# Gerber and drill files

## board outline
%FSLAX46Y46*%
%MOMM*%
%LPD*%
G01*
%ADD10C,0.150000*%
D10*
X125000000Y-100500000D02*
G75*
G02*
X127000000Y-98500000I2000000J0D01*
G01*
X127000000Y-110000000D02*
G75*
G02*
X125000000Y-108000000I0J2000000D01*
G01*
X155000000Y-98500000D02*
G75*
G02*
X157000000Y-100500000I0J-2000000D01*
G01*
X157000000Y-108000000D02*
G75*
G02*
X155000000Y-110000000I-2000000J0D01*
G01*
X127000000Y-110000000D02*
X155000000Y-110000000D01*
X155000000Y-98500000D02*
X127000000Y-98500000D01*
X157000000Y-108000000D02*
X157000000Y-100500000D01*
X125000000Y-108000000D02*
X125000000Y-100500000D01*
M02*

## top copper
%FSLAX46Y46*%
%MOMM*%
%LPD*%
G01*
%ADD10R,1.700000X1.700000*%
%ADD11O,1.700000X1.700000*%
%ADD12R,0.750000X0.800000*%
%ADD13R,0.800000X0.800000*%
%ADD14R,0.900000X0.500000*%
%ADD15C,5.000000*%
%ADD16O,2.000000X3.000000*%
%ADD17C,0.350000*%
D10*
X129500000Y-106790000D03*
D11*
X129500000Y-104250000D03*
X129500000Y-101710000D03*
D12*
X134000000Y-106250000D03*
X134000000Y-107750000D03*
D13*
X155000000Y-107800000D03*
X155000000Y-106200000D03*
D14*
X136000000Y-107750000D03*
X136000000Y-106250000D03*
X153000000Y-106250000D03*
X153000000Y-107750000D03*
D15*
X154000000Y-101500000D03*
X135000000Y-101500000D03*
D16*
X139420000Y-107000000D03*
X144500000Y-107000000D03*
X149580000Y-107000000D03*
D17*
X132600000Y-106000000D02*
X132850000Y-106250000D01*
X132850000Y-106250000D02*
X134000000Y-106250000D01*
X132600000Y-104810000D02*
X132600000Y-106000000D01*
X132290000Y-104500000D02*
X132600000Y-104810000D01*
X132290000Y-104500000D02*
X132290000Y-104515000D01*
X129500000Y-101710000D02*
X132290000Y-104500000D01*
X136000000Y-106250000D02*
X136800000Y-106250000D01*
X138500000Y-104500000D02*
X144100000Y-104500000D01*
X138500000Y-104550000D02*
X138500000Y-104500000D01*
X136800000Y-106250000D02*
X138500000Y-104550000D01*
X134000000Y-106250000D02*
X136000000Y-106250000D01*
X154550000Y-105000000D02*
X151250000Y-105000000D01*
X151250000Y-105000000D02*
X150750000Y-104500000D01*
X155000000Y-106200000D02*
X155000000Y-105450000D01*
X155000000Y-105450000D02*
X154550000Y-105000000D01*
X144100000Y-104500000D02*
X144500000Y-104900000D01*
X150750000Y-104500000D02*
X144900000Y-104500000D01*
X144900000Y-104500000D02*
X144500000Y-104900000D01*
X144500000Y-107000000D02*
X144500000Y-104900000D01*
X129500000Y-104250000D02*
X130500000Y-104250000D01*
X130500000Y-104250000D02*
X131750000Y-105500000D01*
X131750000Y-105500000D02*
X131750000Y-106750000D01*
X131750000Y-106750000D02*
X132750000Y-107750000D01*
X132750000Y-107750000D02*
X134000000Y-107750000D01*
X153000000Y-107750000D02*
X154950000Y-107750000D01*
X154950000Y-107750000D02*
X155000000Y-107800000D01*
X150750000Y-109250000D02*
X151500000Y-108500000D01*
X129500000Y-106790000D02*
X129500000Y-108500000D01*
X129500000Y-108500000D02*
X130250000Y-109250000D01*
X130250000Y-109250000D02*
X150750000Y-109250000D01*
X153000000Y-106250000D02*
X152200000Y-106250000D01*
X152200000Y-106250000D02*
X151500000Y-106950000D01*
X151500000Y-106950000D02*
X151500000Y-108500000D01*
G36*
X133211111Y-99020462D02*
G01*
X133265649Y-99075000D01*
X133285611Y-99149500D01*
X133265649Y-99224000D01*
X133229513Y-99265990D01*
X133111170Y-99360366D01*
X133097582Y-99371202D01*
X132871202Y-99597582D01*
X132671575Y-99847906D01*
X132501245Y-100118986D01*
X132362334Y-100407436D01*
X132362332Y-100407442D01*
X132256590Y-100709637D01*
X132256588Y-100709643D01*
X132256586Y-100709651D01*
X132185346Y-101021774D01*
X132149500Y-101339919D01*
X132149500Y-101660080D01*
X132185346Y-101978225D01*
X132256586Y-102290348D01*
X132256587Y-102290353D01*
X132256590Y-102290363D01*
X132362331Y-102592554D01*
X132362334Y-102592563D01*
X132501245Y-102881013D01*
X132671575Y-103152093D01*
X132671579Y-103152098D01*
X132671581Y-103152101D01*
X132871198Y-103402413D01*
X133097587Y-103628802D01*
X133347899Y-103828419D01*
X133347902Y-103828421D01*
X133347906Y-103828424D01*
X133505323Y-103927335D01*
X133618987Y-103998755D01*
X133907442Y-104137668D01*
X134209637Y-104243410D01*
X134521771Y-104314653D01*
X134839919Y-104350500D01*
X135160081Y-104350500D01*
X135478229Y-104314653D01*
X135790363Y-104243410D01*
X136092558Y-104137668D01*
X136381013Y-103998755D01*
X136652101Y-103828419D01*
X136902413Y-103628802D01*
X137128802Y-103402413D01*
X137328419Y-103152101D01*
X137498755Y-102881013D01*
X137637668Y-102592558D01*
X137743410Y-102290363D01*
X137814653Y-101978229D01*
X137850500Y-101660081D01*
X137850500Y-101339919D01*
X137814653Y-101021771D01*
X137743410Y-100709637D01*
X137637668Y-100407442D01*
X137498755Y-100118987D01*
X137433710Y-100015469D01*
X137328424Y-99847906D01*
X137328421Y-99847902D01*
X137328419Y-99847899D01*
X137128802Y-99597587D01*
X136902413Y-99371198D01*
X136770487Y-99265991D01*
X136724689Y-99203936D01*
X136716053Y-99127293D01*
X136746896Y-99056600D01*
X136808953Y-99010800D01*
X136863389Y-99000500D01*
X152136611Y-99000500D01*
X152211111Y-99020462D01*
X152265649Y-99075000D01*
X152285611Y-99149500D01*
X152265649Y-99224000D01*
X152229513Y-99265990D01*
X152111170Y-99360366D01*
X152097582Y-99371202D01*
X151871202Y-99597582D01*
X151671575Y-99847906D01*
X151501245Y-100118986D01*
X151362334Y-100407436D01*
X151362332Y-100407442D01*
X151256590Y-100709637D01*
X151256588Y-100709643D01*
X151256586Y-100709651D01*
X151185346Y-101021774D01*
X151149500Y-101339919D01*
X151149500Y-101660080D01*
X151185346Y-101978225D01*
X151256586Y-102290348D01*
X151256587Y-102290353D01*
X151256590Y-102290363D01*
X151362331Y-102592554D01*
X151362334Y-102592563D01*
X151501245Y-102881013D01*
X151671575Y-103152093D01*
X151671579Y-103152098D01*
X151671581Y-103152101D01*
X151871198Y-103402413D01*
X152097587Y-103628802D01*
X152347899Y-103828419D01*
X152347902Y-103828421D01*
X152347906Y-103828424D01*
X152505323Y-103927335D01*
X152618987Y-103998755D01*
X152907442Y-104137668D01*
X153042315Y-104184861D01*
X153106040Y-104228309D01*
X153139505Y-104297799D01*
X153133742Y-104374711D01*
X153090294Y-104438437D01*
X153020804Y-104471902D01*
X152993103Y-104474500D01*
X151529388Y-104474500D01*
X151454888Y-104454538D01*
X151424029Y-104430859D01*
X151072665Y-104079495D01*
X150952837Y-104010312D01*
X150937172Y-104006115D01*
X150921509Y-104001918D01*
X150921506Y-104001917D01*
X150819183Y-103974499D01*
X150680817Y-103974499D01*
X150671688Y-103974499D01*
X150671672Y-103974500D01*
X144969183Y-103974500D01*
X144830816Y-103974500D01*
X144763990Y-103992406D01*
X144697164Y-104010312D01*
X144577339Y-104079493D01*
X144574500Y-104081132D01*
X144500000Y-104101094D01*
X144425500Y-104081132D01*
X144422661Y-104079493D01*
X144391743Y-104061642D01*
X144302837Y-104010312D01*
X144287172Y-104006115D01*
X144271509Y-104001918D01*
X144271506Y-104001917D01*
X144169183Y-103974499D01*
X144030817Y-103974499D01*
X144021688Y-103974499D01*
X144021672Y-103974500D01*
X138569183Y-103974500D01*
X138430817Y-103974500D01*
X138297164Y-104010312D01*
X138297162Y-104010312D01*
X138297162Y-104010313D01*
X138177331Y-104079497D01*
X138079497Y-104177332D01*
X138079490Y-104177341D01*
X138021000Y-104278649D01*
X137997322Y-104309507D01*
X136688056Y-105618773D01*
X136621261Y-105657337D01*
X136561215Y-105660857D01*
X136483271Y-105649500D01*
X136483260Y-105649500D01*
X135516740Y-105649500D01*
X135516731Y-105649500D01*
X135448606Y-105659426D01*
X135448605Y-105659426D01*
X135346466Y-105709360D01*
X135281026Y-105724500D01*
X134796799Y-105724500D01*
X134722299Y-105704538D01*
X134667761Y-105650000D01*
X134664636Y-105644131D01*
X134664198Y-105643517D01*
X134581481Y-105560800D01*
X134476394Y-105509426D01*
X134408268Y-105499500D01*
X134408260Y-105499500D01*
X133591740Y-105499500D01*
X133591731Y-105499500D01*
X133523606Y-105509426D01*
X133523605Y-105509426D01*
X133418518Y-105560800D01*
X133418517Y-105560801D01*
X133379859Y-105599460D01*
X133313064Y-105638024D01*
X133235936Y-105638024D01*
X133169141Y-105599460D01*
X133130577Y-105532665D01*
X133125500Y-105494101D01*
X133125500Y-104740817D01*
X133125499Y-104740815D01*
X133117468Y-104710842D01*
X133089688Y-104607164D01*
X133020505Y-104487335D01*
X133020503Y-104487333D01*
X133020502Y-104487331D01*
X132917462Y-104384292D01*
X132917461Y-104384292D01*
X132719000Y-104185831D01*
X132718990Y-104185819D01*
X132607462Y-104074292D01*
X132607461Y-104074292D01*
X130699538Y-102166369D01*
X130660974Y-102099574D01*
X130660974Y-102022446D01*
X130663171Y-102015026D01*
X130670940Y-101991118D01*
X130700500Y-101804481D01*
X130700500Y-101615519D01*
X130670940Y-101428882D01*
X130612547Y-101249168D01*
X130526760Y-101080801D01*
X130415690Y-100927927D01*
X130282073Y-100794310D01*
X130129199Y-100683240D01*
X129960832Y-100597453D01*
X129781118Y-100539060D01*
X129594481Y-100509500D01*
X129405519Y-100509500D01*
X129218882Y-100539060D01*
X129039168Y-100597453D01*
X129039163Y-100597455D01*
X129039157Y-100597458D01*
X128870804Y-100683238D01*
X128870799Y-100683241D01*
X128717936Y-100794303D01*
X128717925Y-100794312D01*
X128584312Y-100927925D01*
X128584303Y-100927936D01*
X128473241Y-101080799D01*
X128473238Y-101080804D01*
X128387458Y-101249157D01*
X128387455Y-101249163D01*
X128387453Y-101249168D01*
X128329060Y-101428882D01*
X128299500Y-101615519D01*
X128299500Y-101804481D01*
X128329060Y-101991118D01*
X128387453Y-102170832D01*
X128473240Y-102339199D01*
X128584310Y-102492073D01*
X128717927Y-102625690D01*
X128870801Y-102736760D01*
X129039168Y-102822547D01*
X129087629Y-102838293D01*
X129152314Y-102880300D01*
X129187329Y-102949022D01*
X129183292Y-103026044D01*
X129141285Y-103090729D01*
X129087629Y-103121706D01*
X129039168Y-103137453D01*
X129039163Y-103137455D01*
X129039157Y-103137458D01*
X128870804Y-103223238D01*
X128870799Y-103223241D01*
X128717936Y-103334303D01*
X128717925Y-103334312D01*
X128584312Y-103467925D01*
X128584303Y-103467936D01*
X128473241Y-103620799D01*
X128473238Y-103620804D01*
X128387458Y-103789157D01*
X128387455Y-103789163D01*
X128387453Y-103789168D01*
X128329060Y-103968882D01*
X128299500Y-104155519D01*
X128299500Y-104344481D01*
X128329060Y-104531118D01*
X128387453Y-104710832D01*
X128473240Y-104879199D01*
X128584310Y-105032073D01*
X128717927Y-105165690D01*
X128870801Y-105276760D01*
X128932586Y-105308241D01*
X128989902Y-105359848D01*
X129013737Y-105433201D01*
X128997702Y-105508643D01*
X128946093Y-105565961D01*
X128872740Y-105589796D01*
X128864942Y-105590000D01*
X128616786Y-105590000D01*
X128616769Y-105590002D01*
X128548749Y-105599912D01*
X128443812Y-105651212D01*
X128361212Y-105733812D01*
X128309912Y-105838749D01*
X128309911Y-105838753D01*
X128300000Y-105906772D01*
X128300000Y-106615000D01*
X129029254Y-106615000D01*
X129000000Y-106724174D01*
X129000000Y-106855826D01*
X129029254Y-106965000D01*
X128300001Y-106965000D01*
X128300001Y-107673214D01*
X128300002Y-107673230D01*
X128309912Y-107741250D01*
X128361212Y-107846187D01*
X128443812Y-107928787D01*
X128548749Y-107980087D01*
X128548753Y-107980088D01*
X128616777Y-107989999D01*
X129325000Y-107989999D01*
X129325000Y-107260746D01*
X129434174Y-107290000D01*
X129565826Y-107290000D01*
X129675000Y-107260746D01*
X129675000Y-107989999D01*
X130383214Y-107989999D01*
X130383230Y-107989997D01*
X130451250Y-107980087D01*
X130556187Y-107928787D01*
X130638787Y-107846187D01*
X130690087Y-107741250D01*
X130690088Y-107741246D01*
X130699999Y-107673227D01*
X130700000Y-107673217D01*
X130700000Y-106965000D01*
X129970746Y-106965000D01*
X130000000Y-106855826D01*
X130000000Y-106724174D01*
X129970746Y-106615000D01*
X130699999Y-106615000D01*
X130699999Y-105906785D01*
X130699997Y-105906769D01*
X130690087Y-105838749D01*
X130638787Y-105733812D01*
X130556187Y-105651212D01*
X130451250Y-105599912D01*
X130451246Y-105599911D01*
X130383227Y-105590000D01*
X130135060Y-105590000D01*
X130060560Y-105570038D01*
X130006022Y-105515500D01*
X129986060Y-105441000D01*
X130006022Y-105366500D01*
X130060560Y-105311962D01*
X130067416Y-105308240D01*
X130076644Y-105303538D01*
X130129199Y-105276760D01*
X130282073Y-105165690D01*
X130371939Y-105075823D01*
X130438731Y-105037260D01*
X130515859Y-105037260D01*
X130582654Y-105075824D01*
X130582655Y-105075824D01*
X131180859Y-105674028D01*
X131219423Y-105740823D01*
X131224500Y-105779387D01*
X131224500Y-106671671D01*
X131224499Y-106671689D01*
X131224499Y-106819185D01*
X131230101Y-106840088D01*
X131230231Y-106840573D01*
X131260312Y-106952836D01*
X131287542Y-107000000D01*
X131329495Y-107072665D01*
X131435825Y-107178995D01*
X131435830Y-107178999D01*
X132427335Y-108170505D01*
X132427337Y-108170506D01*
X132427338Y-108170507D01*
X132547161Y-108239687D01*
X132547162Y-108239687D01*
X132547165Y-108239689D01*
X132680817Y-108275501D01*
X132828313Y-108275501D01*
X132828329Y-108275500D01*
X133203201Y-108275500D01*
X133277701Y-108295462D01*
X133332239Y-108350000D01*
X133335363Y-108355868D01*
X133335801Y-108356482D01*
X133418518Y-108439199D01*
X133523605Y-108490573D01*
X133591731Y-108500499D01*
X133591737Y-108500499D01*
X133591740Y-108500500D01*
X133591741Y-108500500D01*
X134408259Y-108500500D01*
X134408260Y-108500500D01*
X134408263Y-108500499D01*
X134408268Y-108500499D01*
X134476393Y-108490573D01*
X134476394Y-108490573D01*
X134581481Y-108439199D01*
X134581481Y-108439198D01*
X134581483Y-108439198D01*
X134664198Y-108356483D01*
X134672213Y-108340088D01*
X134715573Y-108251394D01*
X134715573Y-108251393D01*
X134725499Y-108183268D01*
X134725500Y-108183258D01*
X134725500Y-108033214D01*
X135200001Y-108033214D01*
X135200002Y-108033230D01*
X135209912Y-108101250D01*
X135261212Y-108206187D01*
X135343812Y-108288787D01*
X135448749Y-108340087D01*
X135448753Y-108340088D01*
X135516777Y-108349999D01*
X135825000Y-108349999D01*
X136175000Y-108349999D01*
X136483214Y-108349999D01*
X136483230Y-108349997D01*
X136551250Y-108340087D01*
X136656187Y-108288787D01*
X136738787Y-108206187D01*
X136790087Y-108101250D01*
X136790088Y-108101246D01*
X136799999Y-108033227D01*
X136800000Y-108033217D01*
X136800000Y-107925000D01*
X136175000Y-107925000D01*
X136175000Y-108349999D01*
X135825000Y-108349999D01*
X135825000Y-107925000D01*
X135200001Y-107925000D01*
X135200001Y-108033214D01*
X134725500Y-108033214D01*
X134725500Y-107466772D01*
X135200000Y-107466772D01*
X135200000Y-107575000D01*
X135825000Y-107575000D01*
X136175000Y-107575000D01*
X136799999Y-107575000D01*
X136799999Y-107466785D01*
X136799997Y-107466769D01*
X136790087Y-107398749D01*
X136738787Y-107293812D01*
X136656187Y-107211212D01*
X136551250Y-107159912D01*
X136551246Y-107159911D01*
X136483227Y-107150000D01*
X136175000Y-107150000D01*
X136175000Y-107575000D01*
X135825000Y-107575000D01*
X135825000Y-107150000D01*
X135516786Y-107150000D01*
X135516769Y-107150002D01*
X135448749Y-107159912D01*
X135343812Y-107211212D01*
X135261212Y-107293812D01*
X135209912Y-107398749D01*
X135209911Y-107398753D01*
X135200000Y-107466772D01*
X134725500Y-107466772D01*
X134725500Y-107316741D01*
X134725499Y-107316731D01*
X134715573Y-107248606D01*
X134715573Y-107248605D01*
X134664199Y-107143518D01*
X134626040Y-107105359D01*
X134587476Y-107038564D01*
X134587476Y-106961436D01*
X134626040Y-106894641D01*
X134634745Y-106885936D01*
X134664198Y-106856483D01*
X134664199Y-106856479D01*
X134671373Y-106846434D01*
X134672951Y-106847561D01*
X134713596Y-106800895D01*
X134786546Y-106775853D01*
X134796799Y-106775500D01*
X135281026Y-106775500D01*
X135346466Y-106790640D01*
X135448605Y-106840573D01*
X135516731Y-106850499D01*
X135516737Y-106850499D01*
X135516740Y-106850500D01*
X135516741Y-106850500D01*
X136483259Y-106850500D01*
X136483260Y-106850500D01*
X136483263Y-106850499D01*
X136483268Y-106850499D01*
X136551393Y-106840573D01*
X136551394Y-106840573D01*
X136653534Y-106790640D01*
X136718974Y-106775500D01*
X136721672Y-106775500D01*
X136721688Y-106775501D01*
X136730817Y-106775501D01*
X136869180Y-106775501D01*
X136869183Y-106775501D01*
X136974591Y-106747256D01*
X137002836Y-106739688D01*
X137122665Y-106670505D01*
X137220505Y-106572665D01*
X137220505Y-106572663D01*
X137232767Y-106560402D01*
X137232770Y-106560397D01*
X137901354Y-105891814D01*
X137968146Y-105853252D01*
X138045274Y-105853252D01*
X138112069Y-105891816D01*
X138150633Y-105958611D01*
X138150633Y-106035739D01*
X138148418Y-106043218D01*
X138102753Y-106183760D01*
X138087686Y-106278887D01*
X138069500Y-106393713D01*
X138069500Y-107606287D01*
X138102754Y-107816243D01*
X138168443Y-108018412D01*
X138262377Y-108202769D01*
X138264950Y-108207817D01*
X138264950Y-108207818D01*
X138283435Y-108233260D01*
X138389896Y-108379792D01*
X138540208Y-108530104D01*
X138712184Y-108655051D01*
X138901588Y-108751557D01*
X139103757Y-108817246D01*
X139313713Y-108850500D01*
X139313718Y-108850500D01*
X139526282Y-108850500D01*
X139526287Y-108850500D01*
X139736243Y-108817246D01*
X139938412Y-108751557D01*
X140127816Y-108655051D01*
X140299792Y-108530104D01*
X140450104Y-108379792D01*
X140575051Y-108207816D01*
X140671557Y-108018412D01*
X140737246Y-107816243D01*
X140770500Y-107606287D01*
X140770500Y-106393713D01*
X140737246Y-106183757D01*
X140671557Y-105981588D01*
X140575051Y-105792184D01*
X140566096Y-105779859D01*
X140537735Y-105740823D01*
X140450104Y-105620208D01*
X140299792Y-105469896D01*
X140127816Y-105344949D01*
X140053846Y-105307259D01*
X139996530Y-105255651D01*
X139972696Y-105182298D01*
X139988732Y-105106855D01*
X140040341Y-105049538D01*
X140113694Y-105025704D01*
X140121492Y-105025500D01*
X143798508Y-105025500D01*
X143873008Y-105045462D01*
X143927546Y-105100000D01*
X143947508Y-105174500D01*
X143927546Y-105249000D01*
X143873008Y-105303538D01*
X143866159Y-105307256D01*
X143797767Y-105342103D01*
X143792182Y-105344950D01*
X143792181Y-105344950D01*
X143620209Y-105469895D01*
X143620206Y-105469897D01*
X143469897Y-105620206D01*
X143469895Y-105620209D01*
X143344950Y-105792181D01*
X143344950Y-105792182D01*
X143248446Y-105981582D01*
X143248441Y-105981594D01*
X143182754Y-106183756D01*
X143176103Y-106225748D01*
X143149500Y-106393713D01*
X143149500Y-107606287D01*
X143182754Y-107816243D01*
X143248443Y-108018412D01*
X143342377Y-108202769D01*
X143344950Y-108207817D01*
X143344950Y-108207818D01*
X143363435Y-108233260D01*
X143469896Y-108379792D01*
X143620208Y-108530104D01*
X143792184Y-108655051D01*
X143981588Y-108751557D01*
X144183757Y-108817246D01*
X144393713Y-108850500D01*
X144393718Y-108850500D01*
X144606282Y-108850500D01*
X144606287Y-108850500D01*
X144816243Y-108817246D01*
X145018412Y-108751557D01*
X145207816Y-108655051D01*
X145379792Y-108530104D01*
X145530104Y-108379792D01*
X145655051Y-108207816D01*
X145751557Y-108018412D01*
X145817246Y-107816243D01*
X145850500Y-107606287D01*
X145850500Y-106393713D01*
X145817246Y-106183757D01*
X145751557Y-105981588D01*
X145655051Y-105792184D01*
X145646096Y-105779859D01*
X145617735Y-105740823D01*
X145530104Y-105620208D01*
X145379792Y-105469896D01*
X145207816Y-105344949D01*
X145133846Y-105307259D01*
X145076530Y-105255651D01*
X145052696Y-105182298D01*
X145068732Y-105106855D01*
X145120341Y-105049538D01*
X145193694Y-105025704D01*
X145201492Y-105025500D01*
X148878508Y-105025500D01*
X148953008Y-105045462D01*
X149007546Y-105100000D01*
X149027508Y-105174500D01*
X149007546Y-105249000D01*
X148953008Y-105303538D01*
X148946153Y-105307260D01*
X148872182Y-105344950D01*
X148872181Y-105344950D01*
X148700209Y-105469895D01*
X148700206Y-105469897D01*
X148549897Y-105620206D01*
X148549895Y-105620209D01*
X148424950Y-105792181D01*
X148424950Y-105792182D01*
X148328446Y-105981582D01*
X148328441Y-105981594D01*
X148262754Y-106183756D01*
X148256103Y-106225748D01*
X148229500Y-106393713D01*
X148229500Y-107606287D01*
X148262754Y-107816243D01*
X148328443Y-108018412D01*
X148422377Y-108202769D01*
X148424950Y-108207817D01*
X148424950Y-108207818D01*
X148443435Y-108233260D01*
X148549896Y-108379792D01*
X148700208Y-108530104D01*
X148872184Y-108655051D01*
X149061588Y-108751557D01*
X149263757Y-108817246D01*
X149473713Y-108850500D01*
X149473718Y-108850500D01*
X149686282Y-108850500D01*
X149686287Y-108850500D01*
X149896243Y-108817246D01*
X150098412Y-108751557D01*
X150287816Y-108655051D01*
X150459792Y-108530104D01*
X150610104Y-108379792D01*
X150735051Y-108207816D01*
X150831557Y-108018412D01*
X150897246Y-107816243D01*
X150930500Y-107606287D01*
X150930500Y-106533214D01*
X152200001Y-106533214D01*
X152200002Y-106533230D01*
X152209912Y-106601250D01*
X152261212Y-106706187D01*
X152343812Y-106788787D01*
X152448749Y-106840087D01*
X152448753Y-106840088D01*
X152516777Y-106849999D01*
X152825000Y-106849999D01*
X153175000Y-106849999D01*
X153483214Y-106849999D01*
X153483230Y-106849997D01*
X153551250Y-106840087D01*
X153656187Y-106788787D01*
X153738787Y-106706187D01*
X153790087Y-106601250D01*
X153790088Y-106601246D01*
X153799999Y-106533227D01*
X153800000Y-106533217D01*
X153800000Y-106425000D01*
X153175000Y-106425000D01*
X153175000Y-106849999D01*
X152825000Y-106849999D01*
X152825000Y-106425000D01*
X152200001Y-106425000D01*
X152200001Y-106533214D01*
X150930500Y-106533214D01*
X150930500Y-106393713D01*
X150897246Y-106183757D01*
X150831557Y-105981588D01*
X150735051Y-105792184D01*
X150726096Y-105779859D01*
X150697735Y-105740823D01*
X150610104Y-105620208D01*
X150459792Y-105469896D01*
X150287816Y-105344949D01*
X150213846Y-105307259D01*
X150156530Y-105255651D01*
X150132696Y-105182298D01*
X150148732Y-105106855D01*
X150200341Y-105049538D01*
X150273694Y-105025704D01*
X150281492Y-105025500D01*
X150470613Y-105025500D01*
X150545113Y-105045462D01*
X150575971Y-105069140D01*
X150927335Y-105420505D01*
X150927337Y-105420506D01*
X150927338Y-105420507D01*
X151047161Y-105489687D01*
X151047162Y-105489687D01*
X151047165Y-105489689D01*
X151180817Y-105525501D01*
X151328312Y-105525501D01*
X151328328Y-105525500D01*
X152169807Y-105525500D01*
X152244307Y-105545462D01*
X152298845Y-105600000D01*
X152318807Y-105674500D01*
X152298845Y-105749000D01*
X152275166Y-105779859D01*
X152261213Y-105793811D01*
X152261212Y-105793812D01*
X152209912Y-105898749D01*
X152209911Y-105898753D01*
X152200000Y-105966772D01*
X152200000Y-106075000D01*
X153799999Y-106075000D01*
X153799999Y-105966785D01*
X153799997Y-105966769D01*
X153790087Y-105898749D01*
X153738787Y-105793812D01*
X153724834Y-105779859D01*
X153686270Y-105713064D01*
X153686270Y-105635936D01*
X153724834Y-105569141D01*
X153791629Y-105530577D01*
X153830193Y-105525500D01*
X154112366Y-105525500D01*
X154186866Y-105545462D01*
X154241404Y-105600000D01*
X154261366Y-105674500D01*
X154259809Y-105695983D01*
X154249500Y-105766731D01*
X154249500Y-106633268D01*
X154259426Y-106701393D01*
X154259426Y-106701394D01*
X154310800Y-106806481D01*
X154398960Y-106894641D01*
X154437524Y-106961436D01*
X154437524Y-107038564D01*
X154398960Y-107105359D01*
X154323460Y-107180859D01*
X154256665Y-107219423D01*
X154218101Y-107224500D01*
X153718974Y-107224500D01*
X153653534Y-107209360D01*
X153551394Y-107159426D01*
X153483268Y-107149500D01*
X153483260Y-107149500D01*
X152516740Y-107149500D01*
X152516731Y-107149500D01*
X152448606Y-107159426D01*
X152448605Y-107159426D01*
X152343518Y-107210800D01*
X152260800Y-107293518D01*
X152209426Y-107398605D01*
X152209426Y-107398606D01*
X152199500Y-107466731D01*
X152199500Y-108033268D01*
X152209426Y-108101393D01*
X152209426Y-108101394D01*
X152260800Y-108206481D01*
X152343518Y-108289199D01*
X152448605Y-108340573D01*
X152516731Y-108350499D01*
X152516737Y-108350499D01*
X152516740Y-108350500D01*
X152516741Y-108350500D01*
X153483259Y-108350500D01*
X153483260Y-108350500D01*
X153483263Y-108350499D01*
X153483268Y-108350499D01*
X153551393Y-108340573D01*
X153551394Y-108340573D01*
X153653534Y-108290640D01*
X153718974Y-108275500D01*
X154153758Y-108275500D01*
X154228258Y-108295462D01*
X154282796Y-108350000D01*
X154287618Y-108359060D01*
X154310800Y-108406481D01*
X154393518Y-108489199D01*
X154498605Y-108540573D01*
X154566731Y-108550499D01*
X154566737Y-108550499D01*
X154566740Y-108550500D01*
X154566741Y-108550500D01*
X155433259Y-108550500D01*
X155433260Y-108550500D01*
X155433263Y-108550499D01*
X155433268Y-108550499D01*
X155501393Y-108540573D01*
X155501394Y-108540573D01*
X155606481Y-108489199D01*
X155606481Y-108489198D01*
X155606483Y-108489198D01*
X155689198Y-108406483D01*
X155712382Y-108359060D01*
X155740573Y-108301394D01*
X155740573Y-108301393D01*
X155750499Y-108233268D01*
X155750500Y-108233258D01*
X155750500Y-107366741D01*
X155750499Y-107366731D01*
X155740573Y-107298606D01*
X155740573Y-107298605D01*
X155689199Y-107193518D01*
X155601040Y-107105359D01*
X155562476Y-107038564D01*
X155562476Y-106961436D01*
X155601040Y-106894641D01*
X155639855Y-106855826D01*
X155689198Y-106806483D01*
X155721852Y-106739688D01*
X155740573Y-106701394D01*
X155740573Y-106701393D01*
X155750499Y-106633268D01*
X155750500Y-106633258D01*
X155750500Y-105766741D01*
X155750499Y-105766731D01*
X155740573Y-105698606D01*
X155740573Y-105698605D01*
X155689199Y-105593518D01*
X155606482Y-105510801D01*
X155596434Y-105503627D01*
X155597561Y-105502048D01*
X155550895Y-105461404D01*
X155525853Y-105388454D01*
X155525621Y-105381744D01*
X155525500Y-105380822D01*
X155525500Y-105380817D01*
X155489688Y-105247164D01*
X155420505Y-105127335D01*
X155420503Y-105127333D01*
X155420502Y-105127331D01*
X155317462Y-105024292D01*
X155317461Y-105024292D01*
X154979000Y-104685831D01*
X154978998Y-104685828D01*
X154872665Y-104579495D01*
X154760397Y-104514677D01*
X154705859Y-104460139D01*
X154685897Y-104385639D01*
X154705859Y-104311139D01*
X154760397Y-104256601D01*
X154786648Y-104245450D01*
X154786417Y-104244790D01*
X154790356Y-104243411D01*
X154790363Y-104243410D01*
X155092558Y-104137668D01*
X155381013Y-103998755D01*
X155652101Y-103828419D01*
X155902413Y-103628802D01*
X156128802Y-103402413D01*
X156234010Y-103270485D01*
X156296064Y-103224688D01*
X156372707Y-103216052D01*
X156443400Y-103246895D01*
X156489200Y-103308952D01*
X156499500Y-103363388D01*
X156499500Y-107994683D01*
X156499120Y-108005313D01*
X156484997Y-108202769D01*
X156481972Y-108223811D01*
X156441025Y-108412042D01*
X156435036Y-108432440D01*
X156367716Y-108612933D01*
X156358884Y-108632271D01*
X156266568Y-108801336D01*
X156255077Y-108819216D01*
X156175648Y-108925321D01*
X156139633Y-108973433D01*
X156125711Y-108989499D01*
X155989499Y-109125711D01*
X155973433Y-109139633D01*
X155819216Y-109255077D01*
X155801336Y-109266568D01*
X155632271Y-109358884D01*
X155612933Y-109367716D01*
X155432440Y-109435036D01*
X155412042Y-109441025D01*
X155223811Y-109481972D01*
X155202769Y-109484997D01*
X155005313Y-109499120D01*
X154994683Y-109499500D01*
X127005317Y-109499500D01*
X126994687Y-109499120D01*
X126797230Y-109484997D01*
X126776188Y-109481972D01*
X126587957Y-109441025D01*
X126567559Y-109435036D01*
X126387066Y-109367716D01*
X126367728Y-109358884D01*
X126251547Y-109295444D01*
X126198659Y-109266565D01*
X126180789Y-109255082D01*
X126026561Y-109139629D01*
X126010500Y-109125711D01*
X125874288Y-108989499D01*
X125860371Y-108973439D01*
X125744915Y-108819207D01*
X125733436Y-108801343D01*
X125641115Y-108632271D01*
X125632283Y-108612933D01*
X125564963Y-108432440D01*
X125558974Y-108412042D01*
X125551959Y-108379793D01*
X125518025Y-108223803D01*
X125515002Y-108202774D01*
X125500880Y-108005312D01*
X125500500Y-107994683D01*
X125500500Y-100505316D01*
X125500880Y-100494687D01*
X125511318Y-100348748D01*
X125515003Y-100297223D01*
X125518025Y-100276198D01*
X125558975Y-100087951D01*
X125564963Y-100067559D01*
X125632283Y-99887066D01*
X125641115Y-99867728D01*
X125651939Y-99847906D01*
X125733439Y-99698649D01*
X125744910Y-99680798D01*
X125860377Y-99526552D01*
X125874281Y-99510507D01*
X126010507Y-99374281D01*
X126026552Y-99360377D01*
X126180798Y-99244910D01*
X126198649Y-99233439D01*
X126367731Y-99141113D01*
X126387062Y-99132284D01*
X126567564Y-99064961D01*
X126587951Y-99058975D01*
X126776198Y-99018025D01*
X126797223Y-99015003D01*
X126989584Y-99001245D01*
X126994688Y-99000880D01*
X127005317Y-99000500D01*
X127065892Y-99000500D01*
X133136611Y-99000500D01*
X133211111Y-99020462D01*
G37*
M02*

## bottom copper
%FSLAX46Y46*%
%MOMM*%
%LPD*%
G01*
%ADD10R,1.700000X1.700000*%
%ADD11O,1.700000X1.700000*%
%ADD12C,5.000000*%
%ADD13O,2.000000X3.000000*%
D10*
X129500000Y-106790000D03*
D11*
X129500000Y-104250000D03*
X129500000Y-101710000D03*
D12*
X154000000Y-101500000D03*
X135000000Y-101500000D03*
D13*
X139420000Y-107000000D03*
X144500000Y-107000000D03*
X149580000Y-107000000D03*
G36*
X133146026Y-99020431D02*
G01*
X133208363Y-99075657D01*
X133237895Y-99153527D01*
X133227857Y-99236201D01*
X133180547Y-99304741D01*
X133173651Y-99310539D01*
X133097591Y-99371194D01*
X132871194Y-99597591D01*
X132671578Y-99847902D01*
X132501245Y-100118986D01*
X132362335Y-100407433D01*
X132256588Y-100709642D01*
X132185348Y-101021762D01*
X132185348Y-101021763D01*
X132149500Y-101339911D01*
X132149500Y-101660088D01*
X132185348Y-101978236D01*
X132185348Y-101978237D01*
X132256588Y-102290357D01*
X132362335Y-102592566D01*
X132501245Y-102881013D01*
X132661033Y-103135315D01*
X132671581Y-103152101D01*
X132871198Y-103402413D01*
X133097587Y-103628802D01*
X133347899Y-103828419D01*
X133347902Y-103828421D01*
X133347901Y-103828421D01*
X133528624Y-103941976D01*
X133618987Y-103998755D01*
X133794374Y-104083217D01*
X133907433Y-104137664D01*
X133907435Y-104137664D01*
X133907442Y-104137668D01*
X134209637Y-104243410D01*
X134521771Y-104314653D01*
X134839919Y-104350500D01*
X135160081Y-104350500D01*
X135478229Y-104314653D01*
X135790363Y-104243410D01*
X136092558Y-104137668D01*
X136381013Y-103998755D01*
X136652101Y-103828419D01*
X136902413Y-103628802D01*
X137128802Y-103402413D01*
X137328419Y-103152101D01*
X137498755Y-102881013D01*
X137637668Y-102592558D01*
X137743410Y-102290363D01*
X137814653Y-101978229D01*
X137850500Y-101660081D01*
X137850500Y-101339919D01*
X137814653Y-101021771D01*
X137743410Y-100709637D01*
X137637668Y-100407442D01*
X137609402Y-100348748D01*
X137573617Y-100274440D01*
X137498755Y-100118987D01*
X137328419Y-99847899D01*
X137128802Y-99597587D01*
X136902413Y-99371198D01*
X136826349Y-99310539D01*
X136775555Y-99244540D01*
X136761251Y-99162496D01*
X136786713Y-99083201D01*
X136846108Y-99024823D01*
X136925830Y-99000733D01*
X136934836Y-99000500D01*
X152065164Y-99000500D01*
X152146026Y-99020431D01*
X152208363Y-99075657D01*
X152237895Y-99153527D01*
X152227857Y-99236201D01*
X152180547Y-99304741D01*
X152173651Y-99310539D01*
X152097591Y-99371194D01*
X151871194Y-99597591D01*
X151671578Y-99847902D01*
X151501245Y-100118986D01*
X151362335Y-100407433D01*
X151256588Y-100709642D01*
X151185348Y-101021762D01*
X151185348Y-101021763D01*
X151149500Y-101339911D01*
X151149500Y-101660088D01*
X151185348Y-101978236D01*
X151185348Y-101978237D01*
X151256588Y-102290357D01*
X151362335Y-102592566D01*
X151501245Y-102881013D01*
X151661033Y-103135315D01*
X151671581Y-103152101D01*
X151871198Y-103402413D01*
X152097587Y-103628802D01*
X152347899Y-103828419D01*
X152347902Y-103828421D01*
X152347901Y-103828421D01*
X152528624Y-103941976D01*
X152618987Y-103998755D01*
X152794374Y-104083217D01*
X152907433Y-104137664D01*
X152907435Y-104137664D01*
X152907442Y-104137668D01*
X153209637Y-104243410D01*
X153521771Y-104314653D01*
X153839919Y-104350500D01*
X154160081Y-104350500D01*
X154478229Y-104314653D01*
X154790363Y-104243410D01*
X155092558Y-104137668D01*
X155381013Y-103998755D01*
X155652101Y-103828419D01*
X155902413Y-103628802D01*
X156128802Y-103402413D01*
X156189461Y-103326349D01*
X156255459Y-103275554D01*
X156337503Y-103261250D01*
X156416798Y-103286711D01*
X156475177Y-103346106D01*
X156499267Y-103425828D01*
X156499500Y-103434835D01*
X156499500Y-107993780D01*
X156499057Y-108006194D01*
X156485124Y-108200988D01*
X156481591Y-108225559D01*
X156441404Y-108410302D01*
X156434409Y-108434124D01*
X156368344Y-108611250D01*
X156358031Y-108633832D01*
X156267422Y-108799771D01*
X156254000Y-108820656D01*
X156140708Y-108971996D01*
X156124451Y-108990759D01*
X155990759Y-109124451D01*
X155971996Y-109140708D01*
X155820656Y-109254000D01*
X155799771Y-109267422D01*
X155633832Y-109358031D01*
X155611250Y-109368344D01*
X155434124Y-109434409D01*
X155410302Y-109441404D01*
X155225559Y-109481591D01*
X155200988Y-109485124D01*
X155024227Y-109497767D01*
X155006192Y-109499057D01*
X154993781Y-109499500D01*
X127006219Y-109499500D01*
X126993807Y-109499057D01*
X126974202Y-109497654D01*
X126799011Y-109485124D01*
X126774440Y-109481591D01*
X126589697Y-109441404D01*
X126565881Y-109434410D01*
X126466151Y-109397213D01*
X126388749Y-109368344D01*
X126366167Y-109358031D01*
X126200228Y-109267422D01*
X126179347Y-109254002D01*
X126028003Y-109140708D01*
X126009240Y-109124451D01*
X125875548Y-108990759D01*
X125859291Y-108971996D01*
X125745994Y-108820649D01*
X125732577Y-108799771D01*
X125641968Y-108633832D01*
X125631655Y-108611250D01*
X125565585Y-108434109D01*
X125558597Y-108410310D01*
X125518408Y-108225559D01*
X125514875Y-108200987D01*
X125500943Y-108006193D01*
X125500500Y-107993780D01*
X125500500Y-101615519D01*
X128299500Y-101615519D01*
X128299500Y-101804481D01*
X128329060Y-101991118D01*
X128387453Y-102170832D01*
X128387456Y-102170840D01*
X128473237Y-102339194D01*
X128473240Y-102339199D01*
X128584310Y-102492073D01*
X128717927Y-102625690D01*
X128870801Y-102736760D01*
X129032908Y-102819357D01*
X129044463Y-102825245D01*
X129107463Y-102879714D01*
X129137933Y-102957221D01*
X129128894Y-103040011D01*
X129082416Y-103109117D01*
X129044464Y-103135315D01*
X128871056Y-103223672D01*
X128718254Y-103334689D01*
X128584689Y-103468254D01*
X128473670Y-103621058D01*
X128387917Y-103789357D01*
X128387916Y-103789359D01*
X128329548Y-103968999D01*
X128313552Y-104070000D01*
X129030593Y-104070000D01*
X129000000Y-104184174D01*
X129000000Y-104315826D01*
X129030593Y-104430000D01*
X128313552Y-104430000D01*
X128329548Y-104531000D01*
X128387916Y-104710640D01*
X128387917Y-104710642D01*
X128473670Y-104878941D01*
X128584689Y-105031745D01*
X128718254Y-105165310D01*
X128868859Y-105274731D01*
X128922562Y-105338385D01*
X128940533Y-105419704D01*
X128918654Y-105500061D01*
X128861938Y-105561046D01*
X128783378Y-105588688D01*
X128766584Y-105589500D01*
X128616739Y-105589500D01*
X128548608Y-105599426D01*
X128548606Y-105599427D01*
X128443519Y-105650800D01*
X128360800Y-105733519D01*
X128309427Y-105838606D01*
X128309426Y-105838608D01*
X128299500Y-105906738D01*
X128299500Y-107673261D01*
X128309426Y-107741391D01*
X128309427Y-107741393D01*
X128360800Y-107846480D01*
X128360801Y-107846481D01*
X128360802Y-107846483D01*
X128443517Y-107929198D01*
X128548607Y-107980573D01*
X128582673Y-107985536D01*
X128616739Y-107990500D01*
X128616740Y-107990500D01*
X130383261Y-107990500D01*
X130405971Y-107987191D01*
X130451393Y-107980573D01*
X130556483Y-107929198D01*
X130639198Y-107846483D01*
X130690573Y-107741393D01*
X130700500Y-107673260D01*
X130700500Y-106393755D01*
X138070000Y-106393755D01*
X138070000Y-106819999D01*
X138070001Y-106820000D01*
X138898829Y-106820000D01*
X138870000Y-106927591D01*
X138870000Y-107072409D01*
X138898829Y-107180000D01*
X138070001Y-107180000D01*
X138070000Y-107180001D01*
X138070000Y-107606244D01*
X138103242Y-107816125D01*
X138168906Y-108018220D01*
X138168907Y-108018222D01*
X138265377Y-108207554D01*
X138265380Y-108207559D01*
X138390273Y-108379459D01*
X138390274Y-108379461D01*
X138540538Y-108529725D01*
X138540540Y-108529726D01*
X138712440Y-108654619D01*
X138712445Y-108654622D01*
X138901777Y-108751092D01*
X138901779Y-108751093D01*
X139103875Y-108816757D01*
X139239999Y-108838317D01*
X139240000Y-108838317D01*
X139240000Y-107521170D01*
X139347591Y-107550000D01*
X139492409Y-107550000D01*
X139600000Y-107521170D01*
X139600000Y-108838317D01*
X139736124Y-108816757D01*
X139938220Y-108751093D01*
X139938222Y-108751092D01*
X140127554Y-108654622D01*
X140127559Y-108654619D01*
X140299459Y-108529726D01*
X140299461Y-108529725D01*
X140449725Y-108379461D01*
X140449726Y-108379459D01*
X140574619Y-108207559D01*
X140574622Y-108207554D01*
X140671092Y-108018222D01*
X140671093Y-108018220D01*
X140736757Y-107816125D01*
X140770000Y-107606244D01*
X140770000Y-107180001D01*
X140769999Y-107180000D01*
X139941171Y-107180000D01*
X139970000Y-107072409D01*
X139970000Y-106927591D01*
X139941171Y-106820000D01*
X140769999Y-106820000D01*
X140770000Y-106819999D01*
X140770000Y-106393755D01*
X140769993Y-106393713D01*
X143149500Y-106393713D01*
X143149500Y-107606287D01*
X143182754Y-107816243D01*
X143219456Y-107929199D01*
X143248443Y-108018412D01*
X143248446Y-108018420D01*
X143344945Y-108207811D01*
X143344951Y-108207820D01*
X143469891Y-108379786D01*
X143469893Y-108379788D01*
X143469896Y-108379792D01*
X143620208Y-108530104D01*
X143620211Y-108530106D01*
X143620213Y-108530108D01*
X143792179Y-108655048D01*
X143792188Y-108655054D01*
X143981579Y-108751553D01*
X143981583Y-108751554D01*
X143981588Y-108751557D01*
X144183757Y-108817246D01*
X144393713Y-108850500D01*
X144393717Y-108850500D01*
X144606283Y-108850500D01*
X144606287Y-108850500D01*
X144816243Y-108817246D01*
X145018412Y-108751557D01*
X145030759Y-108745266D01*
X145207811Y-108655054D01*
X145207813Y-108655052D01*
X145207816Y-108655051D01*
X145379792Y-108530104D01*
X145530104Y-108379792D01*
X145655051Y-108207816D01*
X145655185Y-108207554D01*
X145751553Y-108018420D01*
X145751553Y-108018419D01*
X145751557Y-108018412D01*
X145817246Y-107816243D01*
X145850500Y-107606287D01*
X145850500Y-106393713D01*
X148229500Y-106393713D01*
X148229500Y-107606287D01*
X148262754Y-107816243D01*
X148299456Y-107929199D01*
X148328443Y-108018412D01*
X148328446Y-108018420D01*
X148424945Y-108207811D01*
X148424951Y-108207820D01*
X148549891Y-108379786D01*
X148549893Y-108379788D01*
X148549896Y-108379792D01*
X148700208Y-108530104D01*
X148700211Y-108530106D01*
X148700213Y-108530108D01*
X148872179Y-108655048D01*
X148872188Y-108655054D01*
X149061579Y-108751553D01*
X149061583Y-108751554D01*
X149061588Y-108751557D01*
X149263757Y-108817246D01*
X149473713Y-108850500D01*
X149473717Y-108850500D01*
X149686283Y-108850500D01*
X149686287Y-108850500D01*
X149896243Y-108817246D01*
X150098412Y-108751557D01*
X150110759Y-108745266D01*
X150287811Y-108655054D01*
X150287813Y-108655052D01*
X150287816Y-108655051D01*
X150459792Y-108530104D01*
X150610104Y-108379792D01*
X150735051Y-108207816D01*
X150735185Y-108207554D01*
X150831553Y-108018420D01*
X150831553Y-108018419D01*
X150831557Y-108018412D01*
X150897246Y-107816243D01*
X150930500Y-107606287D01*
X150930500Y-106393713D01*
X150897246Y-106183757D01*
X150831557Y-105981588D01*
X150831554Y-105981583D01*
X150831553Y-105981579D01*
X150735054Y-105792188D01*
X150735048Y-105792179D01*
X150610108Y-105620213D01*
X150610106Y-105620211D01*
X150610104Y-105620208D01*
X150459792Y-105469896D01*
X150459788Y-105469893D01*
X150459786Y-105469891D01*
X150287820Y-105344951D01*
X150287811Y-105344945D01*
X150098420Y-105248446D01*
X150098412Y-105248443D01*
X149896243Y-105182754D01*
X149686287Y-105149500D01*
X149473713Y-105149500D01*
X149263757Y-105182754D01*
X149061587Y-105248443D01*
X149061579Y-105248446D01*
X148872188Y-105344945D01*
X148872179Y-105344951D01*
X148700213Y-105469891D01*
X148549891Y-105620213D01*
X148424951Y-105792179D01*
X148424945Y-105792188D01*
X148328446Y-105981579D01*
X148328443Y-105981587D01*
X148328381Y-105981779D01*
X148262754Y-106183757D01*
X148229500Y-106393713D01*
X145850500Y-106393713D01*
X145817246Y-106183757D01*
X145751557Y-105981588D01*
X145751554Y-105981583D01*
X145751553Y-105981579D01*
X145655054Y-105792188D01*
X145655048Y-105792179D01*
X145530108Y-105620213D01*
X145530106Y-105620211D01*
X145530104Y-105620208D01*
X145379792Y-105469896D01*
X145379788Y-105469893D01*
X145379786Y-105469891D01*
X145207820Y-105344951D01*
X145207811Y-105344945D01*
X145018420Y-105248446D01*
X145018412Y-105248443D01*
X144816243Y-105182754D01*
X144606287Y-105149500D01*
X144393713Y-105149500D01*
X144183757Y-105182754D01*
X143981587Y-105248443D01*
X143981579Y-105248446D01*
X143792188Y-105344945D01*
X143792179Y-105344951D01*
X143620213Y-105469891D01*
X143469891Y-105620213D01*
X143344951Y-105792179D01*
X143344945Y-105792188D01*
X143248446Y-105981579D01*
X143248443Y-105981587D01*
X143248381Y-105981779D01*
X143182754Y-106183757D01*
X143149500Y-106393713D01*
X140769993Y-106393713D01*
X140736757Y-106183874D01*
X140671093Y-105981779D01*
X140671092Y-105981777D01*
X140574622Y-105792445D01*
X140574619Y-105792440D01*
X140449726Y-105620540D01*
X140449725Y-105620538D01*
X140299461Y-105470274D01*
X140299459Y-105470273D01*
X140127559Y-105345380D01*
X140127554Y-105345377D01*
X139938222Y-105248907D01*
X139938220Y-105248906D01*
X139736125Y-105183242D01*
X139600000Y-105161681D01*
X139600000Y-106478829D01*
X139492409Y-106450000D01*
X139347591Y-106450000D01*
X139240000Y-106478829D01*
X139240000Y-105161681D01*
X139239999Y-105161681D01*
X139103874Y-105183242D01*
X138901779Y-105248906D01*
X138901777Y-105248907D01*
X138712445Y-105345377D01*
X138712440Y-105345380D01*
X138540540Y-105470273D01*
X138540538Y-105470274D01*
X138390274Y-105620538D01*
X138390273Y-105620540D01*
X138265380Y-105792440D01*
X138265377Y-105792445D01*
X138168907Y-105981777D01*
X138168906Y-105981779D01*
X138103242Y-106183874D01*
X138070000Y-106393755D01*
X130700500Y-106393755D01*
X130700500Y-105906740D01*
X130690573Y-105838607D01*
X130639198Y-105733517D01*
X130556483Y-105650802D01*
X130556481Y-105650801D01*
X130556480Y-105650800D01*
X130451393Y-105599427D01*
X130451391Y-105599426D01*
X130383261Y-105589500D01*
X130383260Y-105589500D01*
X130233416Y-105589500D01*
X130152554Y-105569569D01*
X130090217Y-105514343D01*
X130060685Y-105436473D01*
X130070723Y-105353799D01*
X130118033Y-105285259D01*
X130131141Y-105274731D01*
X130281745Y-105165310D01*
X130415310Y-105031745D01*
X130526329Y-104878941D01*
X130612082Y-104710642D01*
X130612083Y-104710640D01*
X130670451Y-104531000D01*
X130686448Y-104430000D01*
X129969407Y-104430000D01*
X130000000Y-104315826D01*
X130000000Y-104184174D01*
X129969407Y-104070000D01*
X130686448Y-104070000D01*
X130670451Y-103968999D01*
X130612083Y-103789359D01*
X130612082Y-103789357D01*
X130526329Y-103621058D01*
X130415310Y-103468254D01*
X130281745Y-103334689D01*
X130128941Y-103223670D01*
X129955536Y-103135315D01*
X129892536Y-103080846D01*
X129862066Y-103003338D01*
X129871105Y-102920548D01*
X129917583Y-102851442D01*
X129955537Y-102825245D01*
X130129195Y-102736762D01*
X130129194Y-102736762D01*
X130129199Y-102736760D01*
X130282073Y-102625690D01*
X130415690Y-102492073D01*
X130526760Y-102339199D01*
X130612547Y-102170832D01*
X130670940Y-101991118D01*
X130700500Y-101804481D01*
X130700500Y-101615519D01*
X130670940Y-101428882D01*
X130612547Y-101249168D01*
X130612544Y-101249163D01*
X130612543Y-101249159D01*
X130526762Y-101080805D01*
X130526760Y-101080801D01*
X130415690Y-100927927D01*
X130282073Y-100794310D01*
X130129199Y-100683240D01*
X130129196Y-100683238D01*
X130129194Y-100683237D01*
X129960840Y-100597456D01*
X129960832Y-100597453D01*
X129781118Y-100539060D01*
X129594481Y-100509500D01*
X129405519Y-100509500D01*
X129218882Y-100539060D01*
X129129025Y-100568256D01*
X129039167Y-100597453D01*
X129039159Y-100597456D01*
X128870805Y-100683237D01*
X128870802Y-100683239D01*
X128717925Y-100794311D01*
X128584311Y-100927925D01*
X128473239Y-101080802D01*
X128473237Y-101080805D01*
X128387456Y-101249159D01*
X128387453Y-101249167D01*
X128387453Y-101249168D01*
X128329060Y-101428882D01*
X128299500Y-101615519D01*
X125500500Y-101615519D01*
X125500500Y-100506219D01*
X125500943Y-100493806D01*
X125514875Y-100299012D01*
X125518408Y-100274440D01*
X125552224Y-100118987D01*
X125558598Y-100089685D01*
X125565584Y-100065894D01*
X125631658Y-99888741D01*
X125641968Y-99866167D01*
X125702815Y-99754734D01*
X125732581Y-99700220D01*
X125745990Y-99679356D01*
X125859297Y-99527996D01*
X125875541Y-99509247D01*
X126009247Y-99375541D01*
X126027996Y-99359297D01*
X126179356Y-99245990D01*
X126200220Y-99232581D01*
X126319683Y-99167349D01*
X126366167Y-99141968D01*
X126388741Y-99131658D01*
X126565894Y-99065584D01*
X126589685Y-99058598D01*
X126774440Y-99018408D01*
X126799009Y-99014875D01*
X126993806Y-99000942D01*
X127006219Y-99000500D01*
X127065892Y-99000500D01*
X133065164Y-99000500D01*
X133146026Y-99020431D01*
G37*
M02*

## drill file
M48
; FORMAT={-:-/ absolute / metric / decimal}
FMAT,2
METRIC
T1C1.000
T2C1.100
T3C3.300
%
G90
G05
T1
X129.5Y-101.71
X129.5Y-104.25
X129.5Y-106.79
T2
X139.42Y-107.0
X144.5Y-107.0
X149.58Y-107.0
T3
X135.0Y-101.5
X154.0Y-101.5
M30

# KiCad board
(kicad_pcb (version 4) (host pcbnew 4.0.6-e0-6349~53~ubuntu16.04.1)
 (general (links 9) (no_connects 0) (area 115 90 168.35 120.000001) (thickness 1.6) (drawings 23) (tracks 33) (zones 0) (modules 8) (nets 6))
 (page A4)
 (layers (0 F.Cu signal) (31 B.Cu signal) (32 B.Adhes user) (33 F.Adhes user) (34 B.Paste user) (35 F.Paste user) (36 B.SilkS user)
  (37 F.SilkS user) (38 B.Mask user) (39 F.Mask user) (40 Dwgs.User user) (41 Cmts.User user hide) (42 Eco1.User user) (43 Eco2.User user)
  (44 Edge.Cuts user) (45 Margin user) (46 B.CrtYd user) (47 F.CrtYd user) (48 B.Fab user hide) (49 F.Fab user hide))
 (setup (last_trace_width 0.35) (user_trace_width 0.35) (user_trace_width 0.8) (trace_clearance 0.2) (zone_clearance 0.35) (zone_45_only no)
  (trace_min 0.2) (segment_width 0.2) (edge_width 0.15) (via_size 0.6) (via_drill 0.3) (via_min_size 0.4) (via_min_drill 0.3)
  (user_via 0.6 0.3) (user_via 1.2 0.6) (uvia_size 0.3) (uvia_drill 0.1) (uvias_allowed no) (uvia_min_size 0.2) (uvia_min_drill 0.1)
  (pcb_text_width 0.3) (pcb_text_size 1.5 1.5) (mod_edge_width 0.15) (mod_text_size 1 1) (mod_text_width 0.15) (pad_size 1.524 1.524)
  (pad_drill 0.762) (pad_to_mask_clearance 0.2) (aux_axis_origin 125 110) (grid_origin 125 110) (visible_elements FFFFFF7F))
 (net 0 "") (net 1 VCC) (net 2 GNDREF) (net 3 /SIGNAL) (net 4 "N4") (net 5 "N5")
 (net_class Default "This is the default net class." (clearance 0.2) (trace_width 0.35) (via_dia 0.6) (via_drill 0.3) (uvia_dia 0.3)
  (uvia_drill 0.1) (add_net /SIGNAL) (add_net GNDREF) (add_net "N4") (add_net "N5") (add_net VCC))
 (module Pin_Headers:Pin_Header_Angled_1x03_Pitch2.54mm (layer F.Cu) (at 129.5 106.79 180)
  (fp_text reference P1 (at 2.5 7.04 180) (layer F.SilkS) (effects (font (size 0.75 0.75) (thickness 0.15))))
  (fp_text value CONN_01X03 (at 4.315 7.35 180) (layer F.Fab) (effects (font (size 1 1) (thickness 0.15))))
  (pad 1 thru_hole rect (at 0 0 180) (size 1.7 1.7) (drill 1) (layers *.Cu *.Mask) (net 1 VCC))
  (pad 2 thru_hole oval (at 0 2.54 180) (size 1.7 1.7) (drill 1) (layers *.Cu *.Mask) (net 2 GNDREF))
  (pad 3 thru_hole oval (at 0 5.08 180) (size 1.7 1.7) (drill 1) (layers *.Cu *.Mask) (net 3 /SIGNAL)))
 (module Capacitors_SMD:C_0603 (layer F.Cu) (at 134 107 270)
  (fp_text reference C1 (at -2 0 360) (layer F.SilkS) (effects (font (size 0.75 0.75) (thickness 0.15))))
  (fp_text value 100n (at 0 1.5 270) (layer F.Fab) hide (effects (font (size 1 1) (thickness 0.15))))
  (pad 1 smd rect (at -0.75 0 270) (size 0.8 0.75) (layers F.Cu F.Paste F.Mask) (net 3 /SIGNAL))
  (pad 2 smd rect (at 0.75 0 270) (size 0.8 0.75) (layers F.Cu F.Paste F.Mask) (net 2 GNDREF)))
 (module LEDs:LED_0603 (layer F.Cu) (at 155 107 270)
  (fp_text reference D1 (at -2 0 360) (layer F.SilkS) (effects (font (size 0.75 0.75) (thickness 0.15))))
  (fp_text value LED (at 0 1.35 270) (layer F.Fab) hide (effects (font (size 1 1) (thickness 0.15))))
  (pad 2 smd rect (at 0.8 0 90) (size 0.8 0.8) (layers F.Cu F.Paste F.Mask) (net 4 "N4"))
  (pad 1 smd rect (at -0.8 0 90) (size 0.8 0.8) (layers F.Cu F.Paste F.Mask) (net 3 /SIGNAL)))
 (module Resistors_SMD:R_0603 (layer F.Cu) (at 136 107 90)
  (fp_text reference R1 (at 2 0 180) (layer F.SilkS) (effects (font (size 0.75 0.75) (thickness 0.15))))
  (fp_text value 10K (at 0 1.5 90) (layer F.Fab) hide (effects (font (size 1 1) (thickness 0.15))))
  (pad 1 smd rect (at -0.75 0 90) (size 0.5 0.9) (layers F.Cu F.Paste F.Mask) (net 1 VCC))
  (pad 2 smd rect (at 0.75 0 90) (size 0.5 0.9) (layers F.Cu F.Paste F.Mask) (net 3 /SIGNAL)))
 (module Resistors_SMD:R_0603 (layer F.Cu) (at 153 107 270)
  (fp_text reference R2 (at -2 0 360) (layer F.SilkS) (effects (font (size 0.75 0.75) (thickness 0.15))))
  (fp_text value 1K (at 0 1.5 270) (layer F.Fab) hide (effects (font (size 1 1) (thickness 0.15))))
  (pad 1 smd rect (at -0.75 0 270) (size 0.5 0.9) (layers F.Cu F.Paste F.Mask) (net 1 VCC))
  (pad 2 smd rect (at 0.75 0 270) (size 0.5 0.9) (layers F.Cu F.Paste F.Mask) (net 4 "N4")))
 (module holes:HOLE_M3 (layer F.Cu) (at 154 101.5)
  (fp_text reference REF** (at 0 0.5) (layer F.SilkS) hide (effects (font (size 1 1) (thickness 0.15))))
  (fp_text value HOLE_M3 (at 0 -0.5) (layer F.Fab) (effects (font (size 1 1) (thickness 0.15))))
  (pad "" thru_hole circle (at 0 0) (size 5 5) (drill 3.3) (layers *.Cu)))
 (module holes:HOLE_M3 (layer F.Cu) (at 135 101.5)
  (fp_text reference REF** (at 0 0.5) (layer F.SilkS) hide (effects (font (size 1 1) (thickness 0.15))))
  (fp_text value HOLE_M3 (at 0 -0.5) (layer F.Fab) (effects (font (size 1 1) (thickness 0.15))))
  (pad "" thru_hole circle (at 0 0) (size 5 5) (drill 3.3) (layers *.Cu)))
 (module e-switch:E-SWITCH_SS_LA (layer F.Cu) (at 144.5 107)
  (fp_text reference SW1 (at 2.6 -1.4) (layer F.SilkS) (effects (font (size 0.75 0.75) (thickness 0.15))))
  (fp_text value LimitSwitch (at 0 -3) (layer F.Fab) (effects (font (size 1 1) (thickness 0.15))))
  (pad 1 thru_hole oval (at -5.08 0) (size 2 3) (drill 1.1) (layers *.Cu *.Mask) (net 2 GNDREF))
  (pad 2 thru_hole oval (at 0 0) (size 2 3) (drill 1.1) (layers *.Cu *.Mask) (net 3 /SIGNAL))
  (pad 3 thru_hole oval (at 5.08 0) (size 2 3) (drill 1.1) (layers *.Cu *.Mask) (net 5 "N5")))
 (gr_arc (start 127 100.5) (end 125 100.5) (angle 90) (layer Edge.Cuts) (width 0.15))
 (gr_arc (start 127 108) (end 127 110) (angle 90) (layer Edge.Cuts) (width 0.15))
 (gr_arc (start 155 100.5) (end 155 98.5) (angle 90) (layer Edge.Cuts) (width 0.15))
 (gr_arc (start 155 108) (end 157 108) (angle 90) (layer Edge.Cuts) (width 0.15))
 (gr_line (start 127 110) (end 155 110) (layer Edge.Cuts) (width 0.15))
 (gr_line (start 155 98.5) (end 127 98.5) (layer Edge.Cuts) (width 0.15))
 (gr_line (start 157 108) (end 157 100.5) (layer Edge.Cuts) (width 0.15))
 (gr_line (start 125 108) (end 125 100.5) (layer Edge.Cuts) (width 0.15))
 (segment (start 132.6 106) (end 132.85 106.25) (width 0.35) (layer F.Cu) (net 3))
 (segment (start 132.85 106.25) (end 134 106.25) (width 0.35) (layer F.Cu) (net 3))
 (segment (start 132.6 104.81) (end 132.6 106) (width 0.35) (layer F.Cu) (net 3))
 (segment (start 132.29 104.5) (end 132.6 104.81) (width 0.35) (layer F.Cu) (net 3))
 (segment (start 132.29 104.5) (end 132.29 104.515) (width 0.35) (layer F.Cu) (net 3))
 (segment (start 129.5 101.71) (end 132.29 104.5) (width 0.35) (layer F.Cu) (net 3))
 (segment (start 136 106.25) (end 136.8 106.25) (width 0.35) (layer F.Cu) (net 3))
 (segment (start 138.5 104.5) (end 144.1 104.5) (width 0.35) (layer F.Cu) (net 3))
 (segment (start 138.5 104.55) (end 138.5 104.5) (width 0.35) (layer F.Cu) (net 3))
 (segment (start 136.8 106.25) (end 138.5 104.55) (width 0.35) (layer F.Cu) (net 3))
 (segment (start 134 106.25) (end 136 106.25) (width 0.35) (layer F.Cu) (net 3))
 (segment (start 154.55 105) (end 151.25 105) (width 0.35) (layer F.Cu) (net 3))
 (segment (start 151.25 105) (end 150.75 104.5) (width 0.35) (layer F.Cu) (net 3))
 (segment (start 155 106.2) (end 155 105.45) (width 0.35) (layer F.Cu) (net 3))
 (segment (start 155 105.45) (end 154.55 105) (width 0.35) (layer F.Cu) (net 3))
 (segment (start 144.1 104.5) (end 144.5 104.9) (width 0.35) (layer F.Cu) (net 3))
 (segment (start 150.75 104.5) (end 144.9 104.5) (width 0.35) (layer F.Cu) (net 3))
 (segment (start 144.9 104.5) (end 144.5 104.9) (width 0.35) (layer F.Cu) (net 3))
 (segment (start 144.5 107) (end 144.5 104.9) (width 0.35) (layer F.Cu) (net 3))
 (segment (start 129.5 104.25) (end 130.5 104.25) (width 0.35) (layer F.Cu) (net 2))
 (segment (start 130.5 104.25) (end 131.75 105.5) (width 0.35) (layer F.Cu) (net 2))
 (segment (start 131.75 105.5) (end 131.75 106.75) (width 0.35) (layer F.Cu) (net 2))
 (segment (start 131.75 106.75) (end 132.75 107.75) (width 0.35) (layer F.Cu) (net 2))
 (segment (start 132.75 107.75) (end 134 107.75) (width 0.35) (layer F.Cu) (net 2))
 (segment (start 153 107.75) (end 154.95 107.75) (width 0.35) (layer F.Cu) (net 4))
 (segment (start 154.95 107.75) (end 155 107.8) (width 0.35) (layer F.Cu) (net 4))
 (segment (start 150.75 109.25) (end 151.5 108.5) (width 0.35) (layer F.Cu) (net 1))
 (segment (start 129.5 106.79) (end 129.5 108.5) (width 0.35) (layer F.Cu) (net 1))
 (segment (start 129.5 108.5) (end 130.25 109.25) (width 0.35) (layer F.Cu) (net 1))
 (segment (start 130.25 109.25) (end 150.75 109.25) (width 0.35) (layer F.Cu) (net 1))
 (segment (start 153 106.25) (end 152.2 106.25) (width 0.35) (layer F.Cu) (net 1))
 (segment (start 152.2 106.25) (end 151.5 106.95) (width 0.35) (layer F.Cu) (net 1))
 (segment (start 151.5 106.95) (end 151.5 108.5) (width 0.35) (layer F.Cu) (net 1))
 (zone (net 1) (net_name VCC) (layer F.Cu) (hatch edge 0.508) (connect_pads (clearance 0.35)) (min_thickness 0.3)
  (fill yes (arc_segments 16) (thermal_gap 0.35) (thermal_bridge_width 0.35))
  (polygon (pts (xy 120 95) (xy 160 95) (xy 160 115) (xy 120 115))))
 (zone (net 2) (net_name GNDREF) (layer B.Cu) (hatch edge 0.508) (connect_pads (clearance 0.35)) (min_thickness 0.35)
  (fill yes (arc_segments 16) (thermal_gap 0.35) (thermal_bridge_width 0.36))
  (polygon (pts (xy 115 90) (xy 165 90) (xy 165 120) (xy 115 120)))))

